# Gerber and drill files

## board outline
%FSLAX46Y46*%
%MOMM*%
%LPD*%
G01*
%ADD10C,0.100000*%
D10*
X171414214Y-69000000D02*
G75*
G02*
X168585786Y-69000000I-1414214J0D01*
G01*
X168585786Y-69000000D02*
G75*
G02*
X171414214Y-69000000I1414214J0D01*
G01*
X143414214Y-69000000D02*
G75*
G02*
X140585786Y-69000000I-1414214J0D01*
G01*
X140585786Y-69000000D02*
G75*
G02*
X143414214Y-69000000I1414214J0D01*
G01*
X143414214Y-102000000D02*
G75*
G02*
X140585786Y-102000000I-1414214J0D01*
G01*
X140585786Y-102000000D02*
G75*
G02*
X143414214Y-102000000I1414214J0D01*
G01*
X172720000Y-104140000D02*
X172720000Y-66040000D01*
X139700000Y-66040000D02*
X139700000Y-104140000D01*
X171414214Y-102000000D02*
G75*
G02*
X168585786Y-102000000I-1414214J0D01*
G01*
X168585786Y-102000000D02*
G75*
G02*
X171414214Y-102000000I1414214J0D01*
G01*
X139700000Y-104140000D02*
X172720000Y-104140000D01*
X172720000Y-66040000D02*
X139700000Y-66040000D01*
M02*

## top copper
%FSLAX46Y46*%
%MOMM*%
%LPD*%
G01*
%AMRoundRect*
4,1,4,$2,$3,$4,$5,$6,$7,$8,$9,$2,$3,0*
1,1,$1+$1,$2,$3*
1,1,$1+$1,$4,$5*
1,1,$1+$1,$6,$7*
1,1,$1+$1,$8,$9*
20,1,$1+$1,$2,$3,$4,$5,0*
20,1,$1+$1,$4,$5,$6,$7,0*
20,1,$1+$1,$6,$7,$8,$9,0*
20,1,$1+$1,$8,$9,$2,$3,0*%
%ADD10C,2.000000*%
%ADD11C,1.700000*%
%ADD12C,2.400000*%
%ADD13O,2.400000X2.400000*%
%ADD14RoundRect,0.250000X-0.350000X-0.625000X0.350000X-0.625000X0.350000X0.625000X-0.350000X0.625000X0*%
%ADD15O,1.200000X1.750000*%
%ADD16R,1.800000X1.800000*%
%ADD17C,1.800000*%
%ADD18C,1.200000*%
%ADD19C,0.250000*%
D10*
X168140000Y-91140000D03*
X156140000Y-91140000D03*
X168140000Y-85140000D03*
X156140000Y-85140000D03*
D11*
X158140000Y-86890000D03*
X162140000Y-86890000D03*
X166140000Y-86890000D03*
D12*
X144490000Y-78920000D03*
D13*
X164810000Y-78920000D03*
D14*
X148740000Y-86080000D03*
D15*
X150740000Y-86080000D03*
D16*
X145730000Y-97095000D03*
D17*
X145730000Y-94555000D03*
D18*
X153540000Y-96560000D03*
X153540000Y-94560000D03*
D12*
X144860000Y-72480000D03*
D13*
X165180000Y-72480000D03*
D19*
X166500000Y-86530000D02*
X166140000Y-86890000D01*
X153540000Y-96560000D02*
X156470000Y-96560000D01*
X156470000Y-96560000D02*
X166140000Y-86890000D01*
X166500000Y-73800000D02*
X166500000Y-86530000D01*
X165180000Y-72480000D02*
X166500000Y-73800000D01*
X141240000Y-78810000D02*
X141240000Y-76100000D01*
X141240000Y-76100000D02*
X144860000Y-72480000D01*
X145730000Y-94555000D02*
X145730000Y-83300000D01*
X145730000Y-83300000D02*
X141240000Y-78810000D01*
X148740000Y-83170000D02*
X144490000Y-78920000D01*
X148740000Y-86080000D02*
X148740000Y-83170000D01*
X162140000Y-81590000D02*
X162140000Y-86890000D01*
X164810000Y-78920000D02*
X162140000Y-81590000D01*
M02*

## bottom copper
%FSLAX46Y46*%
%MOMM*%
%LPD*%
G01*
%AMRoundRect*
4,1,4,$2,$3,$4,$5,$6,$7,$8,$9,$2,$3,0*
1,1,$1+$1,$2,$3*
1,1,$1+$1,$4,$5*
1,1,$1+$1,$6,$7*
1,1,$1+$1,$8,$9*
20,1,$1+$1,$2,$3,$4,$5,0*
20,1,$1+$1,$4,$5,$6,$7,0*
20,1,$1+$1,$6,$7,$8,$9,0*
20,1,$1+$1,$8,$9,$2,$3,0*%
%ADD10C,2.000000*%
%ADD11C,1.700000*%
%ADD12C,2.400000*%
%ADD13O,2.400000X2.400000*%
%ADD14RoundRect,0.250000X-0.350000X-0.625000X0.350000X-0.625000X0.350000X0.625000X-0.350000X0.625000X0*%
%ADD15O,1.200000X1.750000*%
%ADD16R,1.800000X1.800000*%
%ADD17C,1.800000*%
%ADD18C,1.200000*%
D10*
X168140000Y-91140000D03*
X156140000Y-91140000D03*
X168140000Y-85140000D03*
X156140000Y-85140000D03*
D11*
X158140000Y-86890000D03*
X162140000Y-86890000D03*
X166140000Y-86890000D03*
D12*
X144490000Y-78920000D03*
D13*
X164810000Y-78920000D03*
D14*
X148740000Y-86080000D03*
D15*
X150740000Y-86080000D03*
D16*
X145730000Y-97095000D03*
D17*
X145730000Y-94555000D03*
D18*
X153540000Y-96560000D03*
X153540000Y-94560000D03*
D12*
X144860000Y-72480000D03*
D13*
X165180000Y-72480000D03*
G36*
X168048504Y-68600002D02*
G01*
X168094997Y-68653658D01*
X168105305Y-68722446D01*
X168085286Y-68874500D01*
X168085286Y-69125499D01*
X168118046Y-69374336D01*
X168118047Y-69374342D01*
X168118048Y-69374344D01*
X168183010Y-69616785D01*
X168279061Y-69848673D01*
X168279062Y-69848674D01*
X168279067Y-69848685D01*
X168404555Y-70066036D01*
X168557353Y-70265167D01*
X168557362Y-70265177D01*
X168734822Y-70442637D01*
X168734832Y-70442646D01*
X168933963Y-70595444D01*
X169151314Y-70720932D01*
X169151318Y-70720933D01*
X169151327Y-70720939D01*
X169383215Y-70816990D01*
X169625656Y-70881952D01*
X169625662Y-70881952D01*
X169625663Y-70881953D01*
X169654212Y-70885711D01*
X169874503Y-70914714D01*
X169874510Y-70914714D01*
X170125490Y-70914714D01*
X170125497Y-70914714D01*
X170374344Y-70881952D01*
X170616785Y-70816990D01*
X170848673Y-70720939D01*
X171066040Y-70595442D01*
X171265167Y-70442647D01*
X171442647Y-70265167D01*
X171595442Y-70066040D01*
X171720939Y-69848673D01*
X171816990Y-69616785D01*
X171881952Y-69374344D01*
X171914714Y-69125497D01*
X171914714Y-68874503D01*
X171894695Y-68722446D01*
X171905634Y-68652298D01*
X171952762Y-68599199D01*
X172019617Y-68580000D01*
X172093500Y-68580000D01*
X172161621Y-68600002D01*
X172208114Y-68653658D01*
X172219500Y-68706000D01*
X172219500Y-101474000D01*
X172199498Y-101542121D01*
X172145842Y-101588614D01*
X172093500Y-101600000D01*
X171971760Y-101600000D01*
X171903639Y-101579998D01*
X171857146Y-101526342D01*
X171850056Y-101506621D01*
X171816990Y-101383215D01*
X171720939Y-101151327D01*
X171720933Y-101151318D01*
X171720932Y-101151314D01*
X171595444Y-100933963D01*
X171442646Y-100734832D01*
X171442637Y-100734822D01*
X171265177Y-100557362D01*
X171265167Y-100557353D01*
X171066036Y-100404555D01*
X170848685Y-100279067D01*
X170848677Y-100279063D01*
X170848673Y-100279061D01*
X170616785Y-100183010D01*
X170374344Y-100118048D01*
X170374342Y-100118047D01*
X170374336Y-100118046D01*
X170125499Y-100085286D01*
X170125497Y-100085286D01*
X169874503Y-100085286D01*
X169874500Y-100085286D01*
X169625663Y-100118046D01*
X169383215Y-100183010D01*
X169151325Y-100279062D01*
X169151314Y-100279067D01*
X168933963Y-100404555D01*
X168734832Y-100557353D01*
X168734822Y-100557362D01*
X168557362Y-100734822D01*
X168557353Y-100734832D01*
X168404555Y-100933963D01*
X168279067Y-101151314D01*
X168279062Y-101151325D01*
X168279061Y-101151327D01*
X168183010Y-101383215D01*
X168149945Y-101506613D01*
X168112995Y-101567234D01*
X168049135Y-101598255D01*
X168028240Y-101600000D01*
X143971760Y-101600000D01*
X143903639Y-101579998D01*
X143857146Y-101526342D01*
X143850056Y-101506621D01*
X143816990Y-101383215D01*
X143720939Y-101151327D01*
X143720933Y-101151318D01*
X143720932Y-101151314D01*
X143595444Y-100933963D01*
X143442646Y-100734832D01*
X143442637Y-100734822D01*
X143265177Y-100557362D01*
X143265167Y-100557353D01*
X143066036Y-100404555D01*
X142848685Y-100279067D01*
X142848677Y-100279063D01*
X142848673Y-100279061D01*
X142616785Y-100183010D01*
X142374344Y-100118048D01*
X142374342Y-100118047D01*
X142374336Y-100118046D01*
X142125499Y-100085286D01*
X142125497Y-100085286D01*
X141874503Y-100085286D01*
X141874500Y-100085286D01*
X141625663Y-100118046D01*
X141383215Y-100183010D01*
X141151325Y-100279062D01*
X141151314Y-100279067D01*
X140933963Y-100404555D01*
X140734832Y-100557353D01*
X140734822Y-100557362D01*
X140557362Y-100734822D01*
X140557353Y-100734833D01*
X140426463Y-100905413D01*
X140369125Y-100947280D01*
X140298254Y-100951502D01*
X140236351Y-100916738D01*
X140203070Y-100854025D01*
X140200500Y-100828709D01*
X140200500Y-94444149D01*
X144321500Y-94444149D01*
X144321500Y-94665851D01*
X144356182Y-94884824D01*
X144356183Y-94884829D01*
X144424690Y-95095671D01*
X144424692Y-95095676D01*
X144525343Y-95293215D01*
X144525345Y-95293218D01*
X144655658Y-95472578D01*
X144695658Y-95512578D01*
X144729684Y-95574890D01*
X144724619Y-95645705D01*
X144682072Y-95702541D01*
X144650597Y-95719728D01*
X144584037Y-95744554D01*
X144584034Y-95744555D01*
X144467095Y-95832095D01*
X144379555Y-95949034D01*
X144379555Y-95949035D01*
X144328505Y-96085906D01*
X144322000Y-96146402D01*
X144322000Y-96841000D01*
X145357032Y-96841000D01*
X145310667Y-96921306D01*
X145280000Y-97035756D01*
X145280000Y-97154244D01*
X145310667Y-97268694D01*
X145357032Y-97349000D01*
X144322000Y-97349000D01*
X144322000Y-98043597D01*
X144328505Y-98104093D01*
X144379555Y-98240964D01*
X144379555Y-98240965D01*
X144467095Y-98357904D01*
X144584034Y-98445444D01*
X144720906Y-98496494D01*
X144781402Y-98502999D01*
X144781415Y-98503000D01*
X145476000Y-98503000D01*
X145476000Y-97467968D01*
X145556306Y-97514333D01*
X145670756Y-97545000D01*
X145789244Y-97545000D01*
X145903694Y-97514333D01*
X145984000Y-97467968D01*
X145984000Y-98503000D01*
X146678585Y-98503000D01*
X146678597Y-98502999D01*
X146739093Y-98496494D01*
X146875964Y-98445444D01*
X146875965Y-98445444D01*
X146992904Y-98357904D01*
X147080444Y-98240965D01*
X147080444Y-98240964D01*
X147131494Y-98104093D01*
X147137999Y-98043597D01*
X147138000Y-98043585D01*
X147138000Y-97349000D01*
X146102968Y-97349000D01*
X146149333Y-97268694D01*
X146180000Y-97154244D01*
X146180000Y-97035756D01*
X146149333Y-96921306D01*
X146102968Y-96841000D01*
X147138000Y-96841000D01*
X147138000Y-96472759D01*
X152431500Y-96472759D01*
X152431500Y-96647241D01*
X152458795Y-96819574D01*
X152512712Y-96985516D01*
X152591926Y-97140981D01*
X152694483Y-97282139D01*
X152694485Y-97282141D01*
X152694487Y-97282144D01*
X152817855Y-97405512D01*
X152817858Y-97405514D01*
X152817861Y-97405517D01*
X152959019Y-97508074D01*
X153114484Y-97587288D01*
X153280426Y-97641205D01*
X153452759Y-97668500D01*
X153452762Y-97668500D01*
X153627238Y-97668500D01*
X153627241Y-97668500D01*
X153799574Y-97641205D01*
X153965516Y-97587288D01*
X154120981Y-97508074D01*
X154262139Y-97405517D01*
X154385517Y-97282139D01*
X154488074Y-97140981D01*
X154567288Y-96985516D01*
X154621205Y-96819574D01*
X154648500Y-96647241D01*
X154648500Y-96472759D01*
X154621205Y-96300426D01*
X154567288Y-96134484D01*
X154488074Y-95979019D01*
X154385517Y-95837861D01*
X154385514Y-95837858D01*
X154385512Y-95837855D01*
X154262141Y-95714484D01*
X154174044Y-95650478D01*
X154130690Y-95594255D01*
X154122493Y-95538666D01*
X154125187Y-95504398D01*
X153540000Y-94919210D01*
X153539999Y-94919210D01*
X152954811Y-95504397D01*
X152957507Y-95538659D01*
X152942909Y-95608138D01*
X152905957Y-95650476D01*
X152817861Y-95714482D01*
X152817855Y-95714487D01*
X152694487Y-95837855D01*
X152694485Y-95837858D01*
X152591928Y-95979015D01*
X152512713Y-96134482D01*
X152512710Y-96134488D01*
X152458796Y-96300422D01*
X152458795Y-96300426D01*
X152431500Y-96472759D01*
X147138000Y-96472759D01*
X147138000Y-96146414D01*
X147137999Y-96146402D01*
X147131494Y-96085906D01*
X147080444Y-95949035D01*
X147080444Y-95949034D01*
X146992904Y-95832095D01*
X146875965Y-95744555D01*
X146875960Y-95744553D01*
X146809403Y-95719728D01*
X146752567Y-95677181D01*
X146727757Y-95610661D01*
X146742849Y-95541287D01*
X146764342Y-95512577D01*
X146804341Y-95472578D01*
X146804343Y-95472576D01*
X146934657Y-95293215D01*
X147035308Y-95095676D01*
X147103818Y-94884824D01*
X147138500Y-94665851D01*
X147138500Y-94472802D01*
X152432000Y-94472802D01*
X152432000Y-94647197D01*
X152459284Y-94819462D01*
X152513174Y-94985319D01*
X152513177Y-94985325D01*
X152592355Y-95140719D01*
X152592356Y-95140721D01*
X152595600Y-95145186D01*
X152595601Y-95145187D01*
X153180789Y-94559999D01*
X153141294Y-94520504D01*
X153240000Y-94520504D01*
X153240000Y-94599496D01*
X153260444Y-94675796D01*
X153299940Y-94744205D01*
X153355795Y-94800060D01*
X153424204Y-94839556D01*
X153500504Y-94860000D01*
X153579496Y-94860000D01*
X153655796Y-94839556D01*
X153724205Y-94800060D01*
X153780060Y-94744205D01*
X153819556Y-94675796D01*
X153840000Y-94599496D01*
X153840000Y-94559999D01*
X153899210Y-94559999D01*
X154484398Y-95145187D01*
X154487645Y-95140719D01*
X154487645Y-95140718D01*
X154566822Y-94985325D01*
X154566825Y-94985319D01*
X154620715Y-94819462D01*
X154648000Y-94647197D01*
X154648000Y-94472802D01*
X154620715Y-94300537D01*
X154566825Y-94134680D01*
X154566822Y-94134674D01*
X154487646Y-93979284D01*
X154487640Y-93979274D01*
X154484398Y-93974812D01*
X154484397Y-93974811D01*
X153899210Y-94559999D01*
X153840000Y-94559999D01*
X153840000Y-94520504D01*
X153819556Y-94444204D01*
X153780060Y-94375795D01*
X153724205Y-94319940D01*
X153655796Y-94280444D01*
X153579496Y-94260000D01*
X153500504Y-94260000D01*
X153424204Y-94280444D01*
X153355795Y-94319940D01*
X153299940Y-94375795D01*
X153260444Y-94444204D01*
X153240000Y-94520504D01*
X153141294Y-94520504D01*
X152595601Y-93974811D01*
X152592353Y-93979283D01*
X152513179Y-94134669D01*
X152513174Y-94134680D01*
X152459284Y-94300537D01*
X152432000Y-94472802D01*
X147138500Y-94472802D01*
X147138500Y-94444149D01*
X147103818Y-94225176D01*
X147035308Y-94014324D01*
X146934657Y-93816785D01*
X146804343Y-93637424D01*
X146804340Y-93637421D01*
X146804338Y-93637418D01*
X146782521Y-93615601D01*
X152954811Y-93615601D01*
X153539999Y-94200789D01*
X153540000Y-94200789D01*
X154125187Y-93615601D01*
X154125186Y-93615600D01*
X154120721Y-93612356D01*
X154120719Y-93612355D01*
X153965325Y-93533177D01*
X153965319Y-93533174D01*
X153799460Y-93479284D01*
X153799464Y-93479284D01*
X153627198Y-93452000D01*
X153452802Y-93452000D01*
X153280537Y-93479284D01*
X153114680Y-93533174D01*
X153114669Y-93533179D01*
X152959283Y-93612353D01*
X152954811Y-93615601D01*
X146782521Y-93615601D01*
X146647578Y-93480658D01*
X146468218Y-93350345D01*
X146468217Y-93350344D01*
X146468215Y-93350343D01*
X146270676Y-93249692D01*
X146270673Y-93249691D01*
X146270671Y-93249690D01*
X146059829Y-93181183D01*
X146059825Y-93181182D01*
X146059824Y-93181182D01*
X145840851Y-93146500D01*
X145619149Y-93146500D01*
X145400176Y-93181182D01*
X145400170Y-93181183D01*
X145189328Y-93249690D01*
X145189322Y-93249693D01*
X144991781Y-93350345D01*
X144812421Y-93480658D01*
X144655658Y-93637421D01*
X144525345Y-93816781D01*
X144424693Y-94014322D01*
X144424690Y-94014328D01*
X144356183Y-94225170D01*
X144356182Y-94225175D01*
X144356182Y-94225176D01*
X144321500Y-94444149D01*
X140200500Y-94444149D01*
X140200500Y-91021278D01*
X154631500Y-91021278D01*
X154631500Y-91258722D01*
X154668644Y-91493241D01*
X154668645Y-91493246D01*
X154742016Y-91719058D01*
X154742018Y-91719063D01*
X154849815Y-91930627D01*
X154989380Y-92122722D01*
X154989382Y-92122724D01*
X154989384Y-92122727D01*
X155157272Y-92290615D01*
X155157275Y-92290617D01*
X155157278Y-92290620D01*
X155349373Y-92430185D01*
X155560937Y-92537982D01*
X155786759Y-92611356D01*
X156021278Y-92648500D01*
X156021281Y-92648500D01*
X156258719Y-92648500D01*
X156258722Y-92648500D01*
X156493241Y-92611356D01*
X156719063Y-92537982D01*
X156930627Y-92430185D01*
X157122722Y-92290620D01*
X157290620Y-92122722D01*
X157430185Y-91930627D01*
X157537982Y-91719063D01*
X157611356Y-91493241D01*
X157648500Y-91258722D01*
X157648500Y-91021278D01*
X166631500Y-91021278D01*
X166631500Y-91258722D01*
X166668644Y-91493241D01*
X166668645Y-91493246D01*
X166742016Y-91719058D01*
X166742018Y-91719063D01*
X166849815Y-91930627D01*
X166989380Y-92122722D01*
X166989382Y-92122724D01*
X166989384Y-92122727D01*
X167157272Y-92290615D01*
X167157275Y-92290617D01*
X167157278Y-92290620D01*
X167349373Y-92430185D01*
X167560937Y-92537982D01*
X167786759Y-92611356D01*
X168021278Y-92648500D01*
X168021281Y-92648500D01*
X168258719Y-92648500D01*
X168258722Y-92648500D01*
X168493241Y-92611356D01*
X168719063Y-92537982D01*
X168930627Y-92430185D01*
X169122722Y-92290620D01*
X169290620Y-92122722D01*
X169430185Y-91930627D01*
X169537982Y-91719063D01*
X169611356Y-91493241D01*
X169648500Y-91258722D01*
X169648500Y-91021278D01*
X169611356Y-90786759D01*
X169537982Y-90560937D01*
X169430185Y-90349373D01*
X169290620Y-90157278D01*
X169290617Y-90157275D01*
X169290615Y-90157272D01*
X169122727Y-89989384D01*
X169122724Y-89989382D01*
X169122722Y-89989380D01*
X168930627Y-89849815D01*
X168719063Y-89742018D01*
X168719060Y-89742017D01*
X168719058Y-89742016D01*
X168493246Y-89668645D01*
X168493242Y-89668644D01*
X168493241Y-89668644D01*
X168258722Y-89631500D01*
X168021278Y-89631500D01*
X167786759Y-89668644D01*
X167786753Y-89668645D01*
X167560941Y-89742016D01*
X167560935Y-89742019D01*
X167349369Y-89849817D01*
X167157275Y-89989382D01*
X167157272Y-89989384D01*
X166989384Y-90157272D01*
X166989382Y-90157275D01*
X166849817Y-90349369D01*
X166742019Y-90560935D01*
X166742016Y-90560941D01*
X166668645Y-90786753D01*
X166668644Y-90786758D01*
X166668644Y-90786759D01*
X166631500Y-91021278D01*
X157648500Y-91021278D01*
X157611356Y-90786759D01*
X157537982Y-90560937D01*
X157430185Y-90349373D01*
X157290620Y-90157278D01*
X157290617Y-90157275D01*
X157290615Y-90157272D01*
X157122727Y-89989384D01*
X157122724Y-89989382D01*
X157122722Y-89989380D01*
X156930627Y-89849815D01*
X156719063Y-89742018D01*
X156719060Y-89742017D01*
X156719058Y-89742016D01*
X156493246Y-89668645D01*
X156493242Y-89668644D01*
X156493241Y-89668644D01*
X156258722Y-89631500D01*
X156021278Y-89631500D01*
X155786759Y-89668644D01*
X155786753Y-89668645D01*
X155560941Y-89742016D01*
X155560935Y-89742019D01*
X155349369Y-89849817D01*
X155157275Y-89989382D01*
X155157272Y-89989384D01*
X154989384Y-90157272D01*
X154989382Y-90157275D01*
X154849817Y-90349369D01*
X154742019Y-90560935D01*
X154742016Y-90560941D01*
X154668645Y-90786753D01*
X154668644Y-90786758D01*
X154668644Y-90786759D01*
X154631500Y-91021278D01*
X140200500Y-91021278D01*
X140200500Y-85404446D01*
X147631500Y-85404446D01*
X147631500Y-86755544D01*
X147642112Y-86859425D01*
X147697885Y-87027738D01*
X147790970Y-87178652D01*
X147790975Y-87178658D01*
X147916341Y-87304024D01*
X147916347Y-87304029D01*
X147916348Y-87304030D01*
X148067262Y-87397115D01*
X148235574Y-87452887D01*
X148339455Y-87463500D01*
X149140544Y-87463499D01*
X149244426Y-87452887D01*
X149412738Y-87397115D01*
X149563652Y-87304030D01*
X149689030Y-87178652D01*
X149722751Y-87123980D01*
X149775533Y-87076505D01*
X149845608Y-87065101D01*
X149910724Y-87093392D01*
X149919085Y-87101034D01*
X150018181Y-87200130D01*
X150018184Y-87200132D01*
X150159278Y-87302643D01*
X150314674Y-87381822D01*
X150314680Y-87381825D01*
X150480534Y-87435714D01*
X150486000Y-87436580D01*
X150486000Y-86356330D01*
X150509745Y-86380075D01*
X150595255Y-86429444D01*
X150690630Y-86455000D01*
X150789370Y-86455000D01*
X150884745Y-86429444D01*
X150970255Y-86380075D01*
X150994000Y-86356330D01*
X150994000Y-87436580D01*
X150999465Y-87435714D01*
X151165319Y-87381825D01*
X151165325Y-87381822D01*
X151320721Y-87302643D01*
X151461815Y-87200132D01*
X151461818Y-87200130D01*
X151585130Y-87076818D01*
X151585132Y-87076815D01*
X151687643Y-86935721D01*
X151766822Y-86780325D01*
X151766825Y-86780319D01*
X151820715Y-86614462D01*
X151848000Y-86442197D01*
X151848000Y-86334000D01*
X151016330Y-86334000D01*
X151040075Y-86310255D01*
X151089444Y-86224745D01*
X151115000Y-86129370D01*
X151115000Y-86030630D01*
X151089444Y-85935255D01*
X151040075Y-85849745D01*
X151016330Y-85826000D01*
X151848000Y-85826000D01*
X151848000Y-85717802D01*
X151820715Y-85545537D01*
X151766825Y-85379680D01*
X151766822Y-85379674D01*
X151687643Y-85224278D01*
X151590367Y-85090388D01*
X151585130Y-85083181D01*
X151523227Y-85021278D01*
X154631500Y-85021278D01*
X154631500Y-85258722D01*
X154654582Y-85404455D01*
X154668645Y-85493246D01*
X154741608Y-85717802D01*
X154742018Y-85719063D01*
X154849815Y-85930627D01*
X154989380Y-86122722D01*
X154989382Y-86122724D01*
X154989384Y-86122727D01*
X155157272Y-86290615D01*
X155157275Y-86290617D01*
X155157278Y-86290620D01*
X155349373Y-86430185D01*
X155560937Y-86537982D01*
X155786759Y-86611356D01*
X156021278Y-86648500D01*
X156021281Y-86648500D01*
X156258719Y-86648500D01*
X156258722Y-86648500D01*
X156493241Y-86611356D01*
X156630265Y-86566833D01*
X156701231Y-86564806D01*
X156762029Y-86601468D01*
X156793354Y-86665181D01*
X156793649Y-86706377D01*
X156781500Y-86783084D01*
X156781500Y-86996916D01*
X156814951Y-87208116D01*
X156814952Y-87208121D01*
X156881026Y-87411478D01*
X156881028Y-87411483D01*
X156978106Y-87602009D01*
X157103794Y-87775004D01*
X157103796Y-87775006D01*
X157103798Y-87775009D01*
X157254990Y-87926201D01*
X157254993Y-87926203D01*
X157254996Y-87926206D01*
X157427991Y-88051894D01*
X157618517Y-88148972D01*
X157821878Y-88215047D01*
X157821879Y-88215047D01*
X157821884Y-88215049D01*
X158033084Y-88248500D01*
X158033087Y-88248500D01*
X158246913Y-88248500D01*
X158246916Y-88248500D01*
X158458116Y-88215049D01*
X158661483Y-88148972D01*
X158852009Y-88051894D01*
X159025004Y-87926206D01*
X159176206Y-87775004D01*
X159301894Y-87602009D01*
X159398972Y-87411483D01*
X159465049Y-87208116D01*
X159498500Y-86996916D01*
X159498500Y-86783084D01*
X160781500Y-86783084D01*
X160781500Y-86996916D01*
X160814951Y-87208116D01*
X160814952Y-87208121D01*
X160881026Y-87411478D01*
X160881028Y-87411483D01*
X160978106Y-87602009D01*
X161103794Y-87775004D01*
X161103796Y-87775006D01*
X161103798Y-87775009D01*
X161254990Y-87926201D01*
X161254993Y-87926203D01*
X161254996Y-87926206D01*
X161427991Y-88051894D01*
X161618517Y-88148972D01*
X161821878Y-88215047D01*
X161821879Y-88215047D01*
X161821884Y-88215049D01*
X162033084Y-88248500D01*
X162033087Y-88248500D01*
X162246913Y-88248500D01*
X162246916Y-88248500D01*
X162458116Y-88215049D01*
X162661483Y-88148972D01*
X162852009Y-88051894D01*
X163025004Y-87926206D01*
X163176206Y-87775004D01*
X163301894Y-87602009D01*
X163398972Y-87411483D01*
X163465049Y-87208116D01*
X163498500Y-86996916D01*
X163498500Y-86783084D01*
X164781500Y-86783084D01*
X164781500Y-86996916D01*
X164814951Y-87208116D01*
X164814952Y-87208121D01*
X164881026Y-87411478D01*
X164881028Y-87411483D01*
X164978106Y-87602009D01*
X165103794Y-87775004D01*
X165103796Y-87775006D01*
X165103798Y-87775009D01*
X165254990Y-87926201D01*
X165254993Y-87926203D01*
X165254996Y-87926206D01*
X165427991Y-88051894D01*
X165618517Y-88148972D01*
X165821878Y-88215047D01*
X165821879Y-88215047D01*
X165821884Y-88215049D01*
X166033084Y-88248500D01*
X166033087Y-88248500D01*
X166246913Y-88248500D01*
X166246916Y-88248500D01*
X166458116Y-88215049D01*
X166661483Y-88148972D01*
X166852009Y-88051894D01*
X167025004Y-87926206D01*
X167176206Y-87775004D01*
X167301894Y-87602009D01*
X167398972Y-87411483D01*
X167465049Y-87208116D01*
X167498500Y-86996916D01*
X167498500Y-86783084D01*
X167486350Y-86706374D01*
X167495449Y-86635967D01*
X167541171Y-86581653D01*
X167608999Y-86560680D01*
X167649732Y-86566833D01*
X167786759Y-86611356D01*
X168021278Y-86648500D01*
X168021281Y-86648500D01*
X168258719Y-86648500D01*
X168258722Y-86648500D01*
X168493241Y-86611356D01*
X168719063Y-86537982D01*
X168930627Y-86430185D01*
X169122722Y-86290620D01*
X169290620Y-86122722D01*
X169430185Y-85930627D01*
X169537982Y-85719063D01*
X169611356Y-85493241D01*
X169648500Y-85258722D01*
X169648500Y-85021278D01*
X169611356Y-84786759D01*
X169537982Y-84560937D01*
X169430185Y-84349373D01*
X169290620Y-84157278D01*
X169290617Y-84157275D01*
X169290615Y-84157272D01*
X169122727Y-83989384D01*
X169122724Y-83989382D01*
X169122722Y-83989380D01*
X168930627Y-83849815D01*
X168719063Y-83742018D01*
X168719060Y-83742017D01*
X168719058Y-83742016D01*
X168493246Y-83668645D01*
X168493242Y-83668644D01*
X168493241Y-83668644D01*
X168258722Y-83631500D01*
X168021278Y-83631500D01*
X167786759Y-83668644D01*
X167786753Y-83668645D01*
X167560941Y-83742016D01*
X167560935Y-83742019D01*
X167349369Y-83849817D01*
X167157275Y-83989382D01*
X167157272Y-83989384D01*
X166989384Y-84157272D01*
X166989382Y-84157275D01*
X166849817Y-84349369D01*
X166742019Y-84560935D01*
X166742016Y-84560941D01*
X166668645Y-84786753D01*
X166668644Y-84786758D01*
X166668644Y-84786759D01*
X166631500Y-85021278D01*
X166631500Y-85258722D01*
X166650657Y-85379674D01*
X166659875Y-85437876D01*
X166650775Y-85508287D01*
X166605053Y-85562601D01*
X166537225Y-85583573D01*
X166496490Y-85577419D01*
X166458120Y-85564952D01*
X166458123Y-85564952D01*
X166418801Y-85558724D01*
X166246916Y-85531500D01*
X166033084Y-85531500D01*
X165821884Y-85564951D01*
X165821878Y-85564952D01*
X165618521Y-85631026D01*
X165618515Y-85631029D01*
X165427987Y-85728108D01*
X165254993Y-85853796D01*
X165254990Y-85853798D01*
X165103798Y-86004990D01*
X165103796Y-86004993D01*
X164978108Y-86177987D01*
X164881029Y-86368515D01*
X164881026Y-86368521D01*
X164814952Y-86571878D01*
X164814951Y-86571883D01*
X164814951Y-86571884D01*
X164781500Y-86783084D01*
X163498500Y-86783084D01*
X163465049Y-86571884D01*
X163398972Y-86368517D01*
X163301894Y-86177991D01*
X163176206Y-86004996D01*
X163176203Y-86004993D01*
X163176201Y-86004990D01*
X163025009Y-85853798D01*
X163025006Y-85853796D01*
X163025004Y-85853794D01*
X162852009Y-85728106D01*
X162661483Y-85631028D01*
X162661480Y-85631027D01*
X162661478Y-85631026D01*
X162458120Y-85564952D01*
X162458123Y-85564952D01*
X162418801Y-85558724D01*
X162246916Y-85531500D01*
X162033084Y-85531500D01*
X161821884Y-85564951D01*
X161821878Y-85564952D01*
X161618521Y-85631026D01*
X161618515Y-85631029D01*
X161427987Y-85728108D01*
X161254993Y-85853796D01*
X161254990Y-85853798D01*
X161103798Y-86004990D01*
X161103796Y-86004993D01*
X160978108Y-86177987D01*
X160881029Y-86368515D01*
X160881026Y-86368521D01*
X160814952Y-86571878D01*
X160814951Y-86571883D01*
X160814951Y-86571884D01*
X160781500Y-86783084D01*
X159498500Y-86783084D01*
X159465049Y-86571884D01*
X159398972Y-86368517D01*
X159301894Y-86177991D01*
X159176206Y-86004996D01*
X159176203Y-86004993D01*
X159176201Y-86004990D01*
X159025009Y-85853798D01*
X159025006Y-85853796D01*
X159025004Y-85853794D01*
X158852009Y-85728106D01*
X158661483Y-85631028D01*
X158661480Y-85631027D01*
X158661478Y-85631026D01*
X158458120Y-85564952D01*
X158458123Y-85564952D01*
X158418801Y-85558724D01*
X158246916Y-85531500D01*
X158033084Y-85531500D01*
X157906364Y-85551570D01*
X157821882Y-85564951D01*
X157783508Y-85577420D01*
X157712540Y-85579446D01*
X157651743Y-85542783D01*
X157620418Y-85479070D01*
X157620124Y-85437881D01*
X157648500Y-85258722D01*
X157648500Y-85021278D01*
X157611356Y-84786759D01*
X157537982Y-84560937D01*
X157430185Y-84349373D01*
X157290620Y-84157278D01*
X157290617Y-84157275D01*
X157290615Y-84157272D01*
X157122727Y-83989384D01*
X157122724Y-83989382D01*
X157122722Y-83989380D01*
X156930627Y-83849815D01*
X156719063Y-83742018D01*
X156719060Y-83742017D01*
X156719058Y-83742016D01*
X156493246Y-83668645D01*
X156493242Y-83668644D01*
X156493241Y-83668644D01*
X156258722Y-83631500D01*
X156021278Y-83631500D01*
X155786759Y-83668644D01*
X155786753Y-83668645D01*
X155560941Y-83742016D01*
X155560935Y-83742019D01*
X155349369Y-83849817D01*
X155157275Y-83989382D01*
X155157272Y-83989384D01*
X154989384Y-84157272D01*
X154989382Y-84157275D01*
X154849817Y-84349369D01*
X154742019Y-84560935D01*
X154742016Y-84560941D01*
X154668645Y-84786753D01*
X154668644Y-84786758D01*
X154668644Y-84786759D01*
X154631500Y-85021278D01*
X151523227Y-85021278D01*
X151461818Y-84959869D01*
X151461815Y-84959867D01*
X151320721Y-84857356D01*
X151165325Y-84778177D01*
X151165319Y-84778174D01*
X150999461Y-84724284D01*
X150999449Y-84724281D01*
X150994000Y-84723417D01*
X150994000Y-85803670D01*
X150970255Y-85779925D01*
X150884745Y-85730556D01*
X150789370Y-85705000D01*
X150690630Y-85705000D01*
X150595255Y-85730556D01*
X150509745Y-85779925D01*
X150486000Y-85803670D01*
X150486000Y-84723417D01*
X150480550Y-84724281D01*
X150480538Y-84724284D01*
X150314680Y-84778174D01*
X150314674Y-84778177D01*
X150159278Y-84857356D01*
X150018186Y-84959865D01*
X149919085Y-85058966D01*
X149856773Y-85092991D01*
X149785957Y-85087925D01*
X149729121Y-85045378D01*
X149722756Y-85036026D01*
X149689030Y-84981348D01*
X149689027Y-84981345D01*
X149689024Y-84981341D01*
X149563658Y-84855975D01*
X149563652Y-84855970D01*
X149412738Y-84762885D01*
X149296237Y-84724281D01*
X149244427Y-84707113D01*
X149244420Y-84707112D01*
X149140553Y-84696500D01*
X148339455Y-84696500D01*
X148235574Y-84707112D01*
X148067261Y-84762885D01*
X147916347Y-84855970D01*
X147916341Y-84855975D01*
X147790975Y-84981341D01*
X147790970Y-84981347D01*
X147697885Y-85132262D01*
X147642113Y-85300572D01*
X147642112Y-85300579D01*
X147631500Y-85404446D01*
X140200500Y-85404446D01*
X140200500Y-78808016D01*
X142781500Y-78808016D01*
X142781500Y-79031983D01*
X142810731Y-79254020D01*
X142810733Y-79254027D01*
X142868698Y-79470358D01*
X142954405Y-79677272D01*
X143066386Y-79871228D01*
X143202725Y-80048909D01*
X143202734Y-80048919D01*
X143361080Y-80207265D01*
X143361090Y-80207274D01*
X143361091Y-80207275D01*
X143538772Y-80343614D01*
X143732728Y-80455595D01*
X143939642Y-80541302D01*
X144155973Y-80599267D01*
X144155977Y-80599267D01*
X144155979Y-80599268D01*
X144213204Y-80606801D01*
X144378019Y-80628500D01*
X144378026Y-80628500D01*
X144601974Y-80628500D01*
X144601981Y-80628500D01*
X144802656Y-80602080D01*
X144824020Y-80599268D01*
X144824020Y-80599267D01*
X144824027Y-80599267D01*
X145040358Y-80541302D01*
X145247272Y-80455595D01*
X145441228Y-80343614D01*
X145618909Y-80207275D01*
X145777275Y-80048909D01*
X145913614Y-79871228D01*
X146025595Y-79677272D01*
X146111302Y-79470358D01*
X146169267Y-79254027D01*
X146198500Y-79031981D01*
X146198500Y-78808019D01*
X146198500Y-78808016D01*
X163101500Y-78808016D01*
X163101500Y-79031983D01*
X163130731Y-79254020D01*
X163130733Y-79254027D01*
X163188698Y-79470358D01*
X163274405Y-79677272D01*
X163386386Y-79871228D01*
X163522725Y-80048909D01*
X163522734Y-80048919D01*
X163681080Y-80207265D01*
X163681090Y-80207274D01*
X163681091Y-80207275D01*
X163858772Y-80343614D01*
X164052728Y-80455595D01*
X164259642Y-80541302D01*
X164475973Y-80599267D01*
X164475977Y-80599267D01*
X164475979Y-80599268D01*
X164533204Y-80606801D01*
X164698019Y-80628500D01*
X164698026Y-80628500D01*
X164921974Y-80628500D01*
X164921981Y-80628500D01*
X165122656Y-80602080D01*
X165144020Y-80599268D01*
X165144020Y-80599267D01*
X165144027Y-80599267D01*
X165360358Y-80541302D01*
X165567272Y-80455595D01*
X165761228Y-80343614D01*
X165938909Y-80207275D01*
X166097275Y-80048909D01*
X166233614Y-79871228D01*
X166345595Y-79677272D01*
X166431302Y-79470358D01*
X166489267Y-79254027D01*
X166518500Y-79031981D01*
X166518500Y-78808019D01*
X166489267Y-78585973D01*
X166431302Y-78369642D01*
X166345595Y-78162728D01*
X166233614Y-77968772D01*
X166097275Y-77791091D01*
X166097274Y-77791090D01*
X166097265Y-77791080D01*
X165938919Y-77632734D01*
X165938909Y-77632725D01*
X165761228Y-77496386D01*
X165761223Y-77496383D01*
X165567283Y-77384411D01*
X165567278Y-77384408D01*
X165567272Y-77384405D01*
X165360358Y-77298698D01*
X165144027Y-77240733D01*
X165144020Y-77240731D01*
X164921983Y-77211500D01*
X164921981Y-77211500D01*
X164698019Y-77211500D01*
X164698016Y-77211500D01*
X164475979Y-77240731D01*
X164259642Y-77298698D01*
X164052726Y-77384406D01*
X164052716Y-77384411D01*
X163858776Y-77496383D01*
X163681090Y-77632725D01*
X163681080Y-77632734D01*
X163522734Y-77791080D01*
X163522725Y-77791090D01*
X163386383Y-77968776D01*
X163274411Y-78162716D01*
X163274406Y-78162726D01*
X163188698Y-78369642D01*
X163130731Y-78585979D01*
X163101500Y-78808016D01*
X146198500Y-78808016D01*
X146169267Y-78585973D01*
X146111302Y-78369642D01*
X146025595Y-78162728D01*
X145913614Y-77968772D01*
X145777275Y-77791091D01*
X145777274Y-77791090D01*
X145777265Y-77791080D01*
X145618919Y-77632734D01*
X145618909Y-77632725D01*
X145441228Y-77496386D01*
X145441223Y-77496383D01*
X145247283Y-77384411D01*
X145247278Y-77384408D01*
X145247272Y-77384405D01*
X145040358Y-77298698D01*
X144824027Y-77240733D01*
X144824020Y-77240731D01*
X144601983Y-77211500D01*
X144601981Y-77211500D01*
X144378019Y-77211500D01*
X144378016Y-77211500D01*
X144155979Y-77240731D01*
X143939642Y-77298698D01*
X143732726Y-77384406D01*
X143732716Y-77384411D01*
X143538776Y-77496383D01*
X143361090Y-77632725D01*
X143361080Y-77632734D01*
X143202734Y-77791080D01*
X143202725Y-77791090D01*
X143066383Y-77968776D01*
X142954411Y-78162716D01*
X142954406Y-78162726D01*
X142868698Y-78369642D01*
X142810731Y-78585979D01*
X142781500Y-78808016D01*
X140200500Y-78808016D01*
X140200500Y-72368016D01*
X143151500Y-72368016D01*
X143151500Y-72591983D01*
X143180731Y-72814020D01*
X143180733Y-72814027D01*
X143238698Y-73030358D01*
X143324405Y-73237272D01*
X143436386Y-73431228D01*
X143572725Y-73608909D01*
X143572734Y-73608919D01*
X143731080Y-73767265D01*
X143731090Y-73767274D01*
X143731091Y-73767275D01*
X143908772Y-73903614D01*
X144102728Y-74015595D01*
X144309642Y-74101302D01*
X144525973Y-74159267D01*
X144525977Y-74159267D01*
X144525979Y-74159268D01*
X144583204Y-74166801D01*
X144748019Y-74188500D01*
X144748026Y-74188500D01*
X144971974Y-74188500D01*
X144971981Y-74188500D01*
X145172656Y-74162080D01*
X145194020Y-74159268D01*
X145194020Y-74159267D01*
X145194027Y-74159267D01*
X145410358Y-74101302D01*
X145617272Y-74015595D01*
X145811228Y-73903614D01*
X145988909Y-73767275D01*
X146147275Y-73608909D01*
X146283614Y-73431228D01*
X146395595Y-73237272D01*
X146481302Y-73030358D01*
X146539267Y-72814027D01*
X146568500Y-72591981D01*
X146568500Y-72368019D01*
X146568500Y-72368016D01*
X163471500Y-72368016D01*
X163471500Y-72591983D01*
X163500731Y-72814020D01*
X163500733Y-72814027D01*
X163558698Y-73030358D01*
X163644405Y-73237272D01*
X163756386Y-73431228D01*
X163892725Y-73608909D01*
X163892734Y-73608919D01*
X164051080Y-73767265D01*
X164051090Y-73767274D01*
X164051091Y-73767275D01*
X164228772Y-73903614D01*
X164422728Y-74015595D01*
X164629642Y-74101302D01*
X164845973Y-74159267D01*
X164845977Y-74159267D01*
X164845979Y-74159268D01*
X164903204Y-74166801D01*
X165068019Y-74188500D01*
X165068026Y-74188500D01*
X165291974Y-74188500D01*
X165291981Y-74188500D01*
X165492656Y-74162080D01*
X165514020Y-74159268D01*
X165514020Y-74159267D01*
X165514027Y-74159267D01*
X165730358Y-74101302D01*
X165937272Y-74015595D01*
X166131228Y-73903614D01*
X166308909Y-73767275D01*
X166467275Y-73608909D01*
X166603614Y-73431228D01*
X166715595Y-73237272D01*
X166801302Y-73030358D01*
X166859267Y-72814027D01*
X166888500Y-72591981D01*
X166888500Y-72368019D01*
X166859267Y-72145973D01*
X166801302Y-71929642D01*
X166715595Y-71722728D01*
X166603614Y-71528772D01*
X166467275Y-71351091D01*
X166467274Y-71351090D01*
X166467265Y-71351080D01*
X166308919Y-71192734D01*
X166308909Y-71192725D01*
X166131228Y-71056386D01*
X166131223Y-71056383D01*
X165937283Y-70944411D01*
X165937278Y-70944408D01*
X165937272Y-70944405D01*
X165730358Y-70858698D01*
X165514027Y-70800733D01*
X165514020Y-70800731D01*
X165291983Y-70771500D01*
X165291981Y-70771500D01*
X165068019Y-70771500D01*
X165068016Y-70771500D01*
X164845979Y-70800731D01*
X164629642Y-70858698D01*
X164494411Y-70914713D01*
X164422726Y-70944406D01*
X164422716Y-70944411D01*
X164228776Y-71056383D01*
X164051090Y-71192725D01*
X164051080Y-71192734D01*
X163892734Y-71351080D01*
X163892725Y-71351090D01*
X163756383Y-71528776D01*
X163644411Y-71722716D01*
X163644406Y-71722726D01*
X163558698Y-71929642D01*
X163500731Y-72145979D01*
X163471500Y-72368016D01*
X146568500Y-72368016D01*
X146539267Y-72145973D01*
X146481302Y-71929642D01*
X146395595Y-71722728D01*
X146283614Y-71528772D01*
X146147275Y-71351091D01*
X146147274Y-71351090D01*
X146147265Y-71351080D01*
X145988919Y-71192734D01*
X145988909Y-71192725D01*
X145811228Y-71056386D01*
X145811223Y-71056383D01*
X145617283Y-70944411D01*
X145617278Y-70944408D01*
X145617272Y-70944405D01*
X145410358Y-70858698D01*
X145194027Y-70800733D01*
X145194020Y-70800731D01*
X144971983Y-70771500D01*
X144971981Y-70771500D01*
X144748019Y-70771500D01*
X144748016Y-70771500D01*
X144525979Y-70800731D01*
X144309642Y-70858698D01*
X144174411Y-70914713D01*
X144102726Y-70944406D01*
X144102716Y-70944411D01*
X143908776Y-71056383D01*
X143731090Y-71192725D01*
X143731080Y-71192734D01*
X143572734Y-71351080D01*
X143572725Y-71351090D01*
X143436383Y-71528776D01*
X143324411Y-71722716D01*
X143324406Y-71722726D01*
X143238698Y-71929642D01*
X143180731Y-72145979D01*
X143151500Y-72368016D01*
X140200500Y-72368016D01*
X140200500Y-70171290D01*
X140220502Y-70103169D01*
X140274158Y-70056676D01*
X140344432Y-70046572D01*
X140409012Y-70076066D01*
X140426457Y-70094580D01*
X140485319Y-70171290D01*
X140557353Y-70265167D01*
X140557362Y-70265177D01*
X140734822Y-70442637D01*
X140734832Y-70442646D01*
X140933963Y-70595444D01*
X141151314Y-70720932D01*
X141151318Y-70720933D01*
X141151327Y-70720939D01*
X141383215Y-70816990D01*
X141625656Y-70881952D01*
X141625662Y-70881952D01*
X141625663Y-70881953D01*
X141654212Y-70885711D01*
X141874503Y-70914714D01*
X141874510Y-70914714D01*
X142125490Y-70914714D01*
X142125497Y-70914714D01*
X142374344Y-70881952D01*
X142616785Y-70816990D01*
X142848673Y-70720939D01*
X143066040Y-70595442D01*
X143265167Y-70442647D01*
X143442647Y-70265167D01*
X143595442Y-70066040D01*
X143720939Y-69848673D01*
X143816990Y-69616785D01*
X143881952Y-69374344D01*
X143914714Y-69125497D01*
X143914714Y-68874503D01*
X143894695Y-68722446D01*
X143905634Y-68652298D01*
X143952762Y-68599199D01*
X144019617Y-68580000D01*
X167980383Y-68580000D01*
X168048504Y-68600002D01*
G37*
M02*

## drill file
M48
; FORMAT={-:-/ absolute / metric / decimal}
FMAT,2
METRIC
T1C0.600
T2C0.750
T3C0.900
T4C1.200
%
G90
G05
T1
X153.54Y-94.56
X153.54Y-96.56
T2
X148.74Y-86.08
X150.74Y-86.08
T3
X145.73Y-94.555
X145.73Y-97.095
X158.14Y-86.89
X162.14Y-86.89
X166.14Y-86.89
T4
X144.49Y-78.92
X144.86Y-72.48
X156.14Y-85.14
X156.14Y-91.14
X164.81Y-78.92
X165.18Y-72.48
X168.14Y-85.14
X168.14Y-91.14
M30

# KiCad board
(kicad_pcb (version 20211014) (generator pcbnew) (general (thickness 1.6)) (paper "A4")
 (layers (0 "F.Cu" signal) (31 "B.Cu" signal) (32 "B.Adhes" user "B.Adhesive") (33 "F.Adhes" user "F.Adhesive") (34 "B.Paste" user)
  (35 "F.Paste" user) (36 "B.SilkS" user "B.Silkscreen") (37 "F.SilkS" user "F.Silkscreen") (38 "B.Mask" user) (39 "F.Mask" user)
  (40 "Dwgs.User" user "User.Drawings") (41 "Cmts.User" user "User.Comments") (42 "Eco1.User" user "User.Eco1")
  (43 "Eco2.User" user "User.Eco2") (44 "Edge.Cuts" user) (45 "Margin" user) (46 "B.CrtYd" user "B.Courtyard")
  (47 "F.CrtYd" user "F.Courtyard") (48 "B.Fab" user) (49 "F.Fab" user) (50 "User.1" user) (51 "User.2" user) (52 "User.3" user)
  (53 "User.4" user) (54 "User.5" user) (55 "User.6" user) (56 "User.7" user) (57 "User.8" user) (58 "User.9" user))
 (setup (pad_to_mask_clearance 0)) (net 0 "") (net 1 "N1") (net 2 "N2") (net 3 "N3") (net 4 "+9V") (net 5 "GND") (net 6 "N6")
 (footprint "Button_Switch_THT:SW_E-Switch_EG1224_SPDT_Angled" (layer "F.Cu") (at 158.14 86.89)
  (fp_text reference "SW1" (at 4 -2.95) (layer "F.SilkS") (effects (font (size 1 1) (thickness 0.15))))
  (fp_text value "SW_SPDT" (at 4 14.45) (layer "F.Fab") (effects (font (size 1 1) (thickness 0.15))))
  (pad "" thru_hole circle (at 10 4.25) (size 2 2) (drill 1.2) (layers *.Cu *.Mask))
  (pad "" thru_hole circle (at -2 4.25) (size 2 2) (drill 1.2) (layers *.Cu *.Mask))
  (pad "" thru_hole circle (at 10 -1.75) (size 2 2) (drill 1.2) (layers *.Cu *.Mask))
  (pad "" thru_hole circle (at -2 -1.75) (size 2 2) (drill 1.2) (layers *.Cu *.Mask))
  (pad "1" thru_hole circle (at 0 0) (size 1.7 1.7) (drill 0.9) (layers *.Cu *.Mask) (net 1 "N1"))
  (pad "2" thru_hole circle (at 4 0) (size 1.7 1.7) (drill 0.9) (layers *.Cu *.Mask) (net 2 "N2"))
  (pad "3" thru_hole circle (at 8 0) (size 1.7 1.7) (drill 0.9) (layers *.Cu *.Mask) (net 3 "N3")))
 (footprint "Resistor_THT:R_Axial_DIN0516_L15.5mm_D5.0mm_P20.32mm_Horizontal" (layer "F.Cu") (at 144.49 78.92)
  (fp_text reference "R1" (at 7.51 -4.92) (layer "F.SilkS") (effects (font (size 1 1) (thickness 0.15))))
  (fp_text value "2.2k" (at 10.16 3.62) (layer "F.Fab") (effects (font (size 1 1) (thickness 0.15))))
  (pad "1" thru_hole circle (at 0 0) (size 2.4 2.4) (drill 1.2) (layers *.Cu *.Mask) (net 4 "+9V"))
  (pad "2" thru_hole oval (at 20.32 0) (size 2.4 2.4) (drill 1.2) (layers *.Cu *.Mask) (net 2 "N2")))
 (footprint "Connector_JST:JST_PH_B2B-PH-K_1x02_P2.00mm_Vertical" (layer "F.Cu") (at 148.74 86.08)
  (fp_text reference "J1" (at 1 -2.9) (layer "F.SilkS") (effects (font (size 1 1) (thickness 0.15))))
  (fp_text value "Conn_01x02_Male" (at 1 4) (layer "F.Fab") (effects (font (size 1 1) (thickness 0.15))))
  (pad "1" thru_hole roundrect (at 0 0) (size 1.2 1.75) (drill 0.75) (layers *.Cu *.Mask) (roundrect_rratio 0.208333) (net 4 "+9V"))
  (pad "2" thru_hole oval (at 2 0) (size 1.2 1.75) (drill 0.75) (layers *.Cu *.Mask) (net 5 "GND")))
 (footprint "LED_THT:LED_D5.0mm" (layer "F.Cu") (at 145.73 97.095 90)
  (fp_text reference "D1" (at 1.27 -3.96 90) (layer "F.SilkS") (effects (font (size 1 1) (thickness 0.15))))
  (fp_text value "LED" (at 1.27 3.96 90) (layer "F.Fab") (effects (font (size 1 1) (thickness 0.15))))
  (pad "1" thru_hole rect (at 0 0 90) (size 1.8 1.8) (drill 0.9) (layers *.Cu *.Mask) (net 5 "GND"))
  (pad "2" thru_hole circle (at 2.54 0 90) (size 1.8 1.8) (drill 0.9) (layers *.Cu *.Mask) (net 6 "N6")))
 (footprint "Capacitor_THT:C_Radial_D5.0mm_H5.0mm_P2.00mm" (layer "F.Cu") (at 153.54 96.56 90)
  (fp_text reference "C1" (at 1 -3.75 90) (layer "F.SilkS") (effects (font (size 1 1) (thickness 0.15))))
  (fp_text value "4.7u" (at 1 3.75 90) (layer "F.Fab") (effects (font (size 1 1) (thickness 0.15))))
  (pad "1" thru_hole circle (at 0 0 90) (size 1.2 1.2) (drill 0.6) (layers *.Cu *.Mask) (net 3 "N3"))
  (pad "2" thru_hole circle (at 2 0 90) (size 1.2 1.2) (drill 0.6) (layers *.Cu *.Mask) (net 5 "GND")))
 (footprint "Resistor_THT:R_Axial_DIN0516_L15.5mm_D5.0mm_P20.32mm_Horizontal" (layer "F.Cu") (at 144.86 72.48)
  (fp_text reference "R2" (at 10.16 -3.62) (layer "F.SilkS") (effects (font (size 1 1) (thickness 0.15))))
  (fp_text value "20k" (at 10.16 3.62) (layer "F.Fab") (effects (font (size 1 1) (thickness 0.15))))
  (pad "1" thru_hole circle (at 0 0) (size 2.4 2.4) (drill 1.2) (layers *.Cu *.Mask) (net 6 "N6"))
  (pad "2" thru_hole oval (at 20.32 0) (size 2.4 2.4) (drill 1.2) (layers *.Cu *.Mask) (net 3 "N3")))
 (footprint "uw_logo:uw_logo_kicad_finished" (layer "F.Cu") (at 148 102)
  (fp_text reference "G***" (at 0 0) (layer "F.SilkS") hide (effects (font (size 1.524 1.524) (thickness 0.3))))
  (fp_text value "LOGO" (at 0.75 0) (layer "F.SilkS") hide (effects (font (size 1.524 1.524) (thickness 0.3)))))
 (gr_circle (center 170 69) (end 169 68) (layer "Edge.Cuts") (width 0.1) (fill none))
 (gr_circle (center 142 69) (end 141 68) (layer "Edge.Cuts") (width 0.1) (fill none))
 (gr_circle (center 142 102) (end 141 103) (layer "Edge.Cuts") (width 0.1) (fill none))
 (gr_line (start 172.72 104.14) (end 172.72 66.04) (layer "Edge.Cuts") (width 0.1))
 (gr_line (start 139.7 66.04) (end 139.7 104.14) (layer "Edge.Cuts") (width 0.1))
 (gr_circle (center 170 102) (end 171 103) (layer "Edge.Cuts") (width 0.1) (fill none))
 (gr_line (start 139.7 104.14) (end 172.72 104.14) (layer "Edge.Cuts") (width 0.1))
 (gr_line (start 172.72 66.04) (end 139.7 66.04) (layer "Edge.Cuts") (width 0.1))
 (segment (start 166.5 86.53) (end 166.14 86.89) (width 0.25) (layer "F.Cu") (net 3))
 (segment (start 153.54 96.56) (end 156.47 96.56) (width 0.25) (layer "F.Cu") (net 3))
 (segment (start 156.47 96.56) (end 166.14 86.89) (width 0.25) (layer "F.Cu") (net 3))
 (segment (start 166.5 73.8) (end 166.5 86.53) (width 0.25) (layer "F.Cu") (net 3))
 (segment (start 165.18 72.48) (end 166.5 73.8) (width 0.25) (layer "F.Cu") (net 3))
 (segment (start 141.24 78.81) (end 141.24 76.1) (width 0.25) (layer "F.Cu") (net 6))
 (segment (start 141.24 76.1) (end 144.86 72.48) (width 0.25) (layer "F.Cu") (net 6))
 (segment (start 145.73 94.555) (end 145.73 83.3) (width 0.25) (layer "F.Cu") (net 6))
 (segment (start 145.73 83.3) (end 141.24 78.81) (width 0.25) (layer "F.Cu") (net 6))
 (segment (start 148.74 83.17) (end 144.49 78.92) (width 0.25) (layer "F.Cu") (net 4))
 (segment (start 148.74 86.08) (end 148.74 83.17) (width 0.25) (layer "F.Cu") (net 4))
 (segment (start 162.14 81.59) (end 162.14 86.89) (width 0.25) (layer "F.Cu") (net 2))
 (segment (start 164.81 78.92) (end 162.14 81.59) (width 0.25) (layer "F.Cu") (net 2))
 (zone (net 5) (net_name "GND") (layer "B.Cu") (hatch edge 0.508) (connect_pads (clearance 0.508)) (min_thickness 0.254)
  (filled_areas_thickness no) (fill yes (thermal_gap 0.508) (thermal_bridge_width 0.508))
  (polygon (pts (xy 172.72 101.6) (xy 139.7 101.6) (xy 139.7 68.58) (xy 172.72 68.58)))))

